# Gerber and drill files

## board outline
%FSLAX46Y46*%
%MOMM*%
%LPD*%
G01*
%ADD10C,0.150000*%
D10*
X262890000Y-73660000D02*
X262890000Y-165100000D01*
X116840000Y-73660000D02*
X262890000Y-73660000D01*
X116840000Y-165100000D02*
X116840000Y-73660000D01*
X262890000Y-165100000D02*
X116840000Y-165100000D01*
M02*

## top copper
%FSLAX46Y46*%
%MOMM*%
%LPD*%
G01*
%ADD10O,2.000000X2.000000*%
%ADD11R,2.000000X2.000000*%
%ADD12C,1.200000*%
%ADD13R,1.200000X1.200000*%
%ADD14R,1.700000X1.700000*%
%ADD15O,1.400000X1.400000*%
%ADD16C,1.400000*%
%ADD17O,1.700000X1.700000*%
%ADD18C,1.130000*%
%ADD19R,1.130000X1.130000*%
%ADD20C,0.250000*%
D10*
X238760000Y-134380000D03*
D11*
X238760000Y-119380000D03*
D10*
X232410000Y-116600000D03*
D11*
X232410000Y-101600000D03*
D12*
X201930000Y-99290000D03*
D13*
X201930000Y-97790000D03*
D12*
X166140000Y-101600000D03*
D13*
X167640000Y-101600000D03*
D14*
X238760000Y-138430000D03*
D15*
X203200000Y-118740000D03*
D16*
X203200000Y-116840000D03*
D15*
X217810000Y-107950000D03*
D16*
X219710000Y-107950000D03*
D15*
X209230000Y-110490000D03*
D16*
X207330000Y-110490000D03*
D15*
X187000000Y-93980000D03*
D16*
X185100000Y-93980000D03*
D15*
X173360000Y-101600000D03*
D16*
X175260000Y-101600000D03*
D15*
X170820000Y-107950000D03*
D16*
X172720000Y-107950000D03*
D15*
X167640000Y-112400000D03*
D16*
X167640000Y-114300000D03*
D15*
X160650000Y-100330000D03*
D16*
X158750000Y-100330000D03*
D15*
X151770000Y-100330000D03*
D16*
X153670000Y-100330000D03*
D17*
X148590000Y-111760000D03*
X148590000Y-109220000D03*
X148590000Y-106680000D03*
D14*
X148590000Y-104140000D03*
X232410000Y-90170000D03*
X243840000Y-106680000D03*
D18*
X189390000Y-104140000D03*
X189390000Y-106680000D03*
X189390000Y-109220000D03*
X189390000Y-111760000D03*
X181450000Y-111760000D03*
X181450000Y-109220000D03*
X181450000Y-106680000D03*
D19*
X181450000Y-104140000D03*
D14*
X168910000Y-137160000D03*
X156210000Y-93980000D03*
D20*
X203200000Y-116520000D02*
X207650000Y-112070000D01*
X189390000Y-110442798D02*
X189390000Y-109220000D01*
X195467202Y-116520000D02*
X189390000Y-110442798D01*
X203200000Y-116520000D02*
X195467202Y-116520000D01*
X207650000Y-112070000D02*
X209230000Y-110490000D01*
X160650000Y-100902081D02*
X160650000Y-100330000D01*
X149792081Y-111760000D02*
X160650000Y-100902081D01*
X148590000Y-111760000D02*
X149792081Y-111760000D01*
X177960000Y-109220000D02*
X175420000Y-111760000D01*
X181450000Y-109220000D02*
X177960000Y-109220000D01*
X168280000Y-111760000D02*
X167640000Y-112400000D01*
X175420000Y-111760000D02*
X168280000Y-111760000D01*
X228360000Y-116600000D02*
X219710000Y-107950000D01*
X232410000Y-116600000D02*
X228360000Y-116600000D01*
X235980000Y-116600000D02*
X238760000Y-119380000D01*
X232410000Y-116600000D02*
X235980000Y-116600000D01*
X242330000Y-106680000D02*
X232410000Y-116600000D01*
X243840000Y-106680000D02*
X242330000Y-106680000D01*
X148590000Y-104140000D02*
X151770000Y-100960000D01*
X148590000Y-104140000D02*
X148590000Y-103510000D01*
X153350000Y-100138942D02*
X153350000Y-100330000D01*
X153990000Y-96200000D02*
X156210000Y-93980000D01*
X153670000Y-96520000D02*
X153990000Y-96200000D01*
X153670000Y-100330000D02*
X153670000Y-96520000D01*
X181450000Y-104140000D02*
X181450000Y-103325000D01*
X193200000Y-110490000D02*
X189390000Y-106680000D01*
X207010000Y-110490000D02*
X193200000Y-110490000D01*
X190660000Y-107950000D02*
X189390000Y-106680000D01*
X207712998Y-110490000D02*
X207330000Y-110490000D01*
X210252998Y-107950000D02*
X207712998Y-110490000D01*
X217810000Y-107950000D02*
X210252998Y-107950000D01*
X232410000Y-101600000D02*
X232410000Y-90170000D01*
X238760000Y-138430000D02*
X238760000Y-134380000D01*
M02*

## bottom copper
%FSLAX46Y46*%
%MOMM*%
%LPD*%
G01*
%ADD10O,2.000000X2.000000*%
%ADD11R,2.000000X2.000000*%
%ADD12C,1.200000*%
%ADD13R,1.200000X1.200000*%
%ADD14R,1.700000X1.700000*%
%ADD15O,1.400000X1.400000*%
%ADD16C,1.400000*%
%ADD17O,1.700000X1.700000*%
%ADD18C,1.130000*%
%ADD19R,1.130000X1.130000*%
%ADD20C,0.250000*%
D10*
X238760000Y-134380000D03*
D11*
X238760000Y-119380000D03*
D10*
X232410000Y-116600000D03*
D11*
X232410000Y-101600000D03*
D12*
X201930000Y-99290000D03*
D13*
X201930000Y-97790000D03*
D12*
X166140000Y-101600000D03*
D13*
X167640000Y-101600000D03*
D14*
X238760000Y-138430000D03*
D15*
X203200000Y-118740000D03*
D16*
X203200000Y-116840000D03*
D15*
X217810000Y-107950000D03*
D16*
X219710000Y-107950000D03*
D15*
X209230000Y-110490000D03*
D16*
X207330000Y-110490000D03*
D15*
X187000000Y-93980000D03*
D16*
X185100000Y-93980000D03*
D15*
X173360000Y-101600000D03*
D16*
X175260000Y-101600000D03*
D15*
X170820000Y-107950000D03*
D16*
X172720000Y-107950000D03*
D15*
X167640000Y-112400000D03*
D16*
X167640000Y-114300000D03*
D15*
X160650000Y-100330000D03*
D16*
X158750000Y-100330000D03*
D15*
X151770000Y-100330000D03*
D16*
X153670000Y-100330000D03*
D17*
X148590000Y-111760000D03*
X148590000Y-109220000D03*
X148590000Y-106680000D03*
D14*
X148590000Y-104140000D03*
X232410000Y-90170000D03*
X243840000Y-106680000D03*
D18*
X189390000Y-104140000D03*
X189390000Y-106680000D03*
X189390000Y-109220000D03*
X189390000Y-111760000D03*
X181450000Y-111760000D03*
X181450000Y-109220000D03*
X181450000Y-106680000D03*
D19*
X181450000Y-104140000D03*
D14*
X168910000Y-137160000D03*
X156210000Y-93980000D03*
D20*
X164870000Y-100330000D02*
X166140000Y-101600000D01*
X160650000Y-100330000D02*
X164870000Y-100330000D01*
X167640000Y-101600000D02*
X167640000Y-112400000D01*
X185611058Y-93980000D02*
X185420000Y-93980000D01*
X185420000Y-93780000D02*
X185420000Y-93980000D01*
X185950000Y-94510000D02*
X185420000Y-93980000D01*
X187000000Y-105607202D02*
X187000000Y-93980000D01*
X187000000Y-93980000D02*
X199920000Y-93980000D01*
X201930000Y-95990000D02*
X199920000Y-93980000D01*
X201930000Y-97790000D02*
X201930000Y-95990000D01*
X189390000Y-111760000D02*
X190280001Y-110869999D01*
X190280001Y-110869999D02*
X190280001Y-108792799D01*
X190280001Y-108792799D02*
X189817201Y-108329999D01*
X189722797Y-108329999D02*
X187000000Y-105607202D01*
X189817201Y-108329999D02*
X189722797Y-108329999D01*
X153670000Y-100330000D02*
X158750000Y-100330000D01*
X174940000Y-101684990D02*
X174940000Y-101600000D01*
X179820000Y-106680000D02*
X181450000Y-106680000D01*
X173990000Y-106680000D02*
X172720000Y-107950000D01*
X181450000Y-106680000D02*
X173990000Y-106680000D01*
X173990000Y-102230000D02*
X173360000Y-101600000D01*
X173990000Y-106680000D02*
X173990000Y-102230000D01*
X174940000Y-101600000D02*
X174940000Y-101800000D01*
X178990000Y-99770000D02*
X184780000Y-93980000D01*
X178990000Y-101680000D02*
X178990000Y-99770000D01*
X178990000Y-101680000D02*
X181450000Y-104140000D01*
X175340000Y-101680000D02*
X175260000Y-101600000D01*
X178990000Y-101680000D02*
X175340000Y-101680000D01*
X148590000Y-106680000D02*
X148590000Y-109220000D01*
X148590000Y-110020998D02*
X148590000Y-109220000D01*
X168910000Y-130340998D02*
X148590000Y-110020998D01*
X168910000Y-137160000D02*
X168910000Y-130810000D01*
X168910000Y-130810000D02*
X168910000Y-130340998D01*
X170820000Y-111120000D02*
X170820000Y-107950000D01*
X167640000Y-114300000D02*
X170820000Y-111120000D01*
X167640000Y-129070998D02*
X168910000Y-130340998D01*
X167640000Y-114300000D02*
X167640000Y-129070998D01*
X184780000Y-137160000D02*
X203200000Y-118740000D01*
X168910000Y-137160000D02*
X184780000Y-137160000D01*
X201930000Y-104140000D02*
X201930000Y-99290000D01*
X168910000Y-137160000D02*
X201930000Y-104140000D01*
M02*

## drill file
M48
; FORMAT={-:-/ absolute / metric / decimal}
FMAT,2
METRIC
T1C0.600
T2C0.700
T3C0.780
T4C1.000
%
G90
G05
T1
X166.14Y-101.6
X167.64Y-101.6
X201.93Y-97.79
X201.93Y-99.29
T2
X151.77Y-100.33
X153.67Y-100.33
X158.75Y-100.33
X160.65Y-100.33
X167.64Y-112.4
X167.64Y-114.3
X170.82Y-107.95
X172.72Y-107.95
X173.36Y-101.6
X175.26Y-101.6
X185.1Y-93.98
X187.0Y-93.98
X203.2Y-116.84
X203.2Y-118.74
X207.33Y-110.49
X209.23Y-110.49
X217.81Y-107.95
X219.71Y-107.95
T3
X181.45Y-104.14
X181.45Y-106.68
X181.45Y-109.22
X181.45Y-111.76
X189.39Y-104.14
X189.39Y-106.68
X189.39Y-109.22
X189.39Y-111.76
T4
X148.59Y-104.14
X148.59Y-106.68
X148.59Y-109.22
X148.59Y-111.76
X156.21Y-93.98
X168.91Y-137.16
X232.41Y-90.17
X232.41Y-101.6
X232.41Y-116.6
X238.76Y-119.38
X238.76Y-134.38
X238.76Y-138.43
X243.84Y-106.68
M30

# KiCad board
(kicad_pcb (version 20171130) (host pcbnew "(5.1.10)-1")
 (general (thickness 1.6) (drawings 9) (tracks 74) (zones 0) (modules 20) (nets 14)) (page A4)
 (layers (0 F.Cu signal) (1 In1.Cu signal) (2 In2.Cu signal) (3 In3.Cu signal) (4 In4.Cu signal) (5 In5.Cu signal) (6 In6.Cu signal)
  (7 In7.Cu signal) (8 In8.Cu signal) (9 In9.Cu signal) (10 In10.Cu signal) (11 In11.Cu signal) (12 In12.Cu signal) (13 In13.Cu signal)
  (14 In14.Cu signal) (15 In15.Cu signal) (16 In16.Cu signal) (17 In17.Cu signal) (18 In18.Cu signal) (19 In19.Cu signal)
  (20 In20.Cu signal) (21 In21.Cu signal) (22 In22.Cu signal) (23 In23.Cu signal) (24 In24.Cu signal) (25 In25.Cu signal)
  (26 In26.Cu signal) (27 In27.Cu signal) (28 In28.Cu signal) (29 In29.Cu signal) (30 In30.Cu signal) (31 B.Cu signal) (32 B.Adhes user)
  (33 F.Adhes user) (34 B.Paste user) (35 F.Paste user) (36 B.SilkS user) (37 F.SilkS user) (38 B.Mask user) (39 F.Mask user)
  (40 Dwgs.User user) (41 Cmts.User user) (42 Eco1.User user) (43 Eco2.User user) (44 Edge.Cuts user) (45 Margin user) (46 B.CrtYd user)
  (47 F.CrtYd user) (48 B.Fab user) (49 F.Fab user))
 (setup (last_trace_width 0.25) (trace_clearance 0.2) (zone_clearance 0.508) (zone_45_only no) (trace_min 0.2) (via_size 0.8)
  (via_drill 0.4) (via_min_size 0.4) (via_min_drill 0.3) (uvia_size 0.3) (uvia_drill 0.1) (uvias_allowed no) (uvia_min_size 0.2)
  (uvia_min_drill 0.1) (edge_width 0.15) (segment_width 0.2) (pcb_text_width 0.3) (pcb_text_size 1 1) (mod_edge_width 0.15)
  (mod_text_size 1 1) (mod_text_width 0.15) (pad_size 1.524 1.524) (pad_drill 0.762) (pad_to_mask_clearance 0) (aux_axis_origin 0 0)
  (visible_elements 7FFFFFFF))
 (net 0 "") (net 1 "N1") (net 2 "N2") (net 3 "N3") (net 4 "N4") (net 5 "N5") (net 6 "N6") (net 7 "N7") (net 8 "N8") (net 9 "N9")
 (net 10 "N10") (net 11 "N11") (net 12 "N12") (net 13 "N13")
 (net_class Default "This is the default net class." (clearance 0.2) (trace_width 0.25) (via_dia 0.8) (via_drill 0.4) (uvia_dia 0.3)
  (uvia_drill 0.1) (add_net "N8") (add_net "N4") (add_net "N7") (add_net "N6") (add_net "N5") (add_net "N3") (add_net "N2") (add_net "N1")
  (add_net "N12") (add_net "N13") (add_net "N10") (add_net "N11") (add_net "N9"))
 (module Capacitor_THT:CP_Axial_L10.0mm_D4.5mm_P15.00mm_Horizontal (layer F.Cu) (at 238.76 119.38 270)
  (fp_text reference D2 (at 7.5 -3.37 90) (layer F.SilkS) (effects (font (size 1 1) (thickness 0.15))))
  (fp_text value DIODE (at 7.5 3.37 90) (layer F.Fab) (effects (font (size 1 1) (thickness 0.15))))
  (pad 2 thru_hole oval (at 15 0 270) (size 2 2) (drill 1) (layers *.Cu *.Mask) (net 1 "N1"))
  (pad 1 thru_hole rect (at 0 0 270) (size 2 2) (drill 1) (layers *.Cu *.Mask) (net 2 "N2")))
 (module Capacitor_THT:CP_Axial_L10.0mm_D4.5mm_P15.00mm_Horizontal (layer F.Cu) (at 232.41 101.6 270)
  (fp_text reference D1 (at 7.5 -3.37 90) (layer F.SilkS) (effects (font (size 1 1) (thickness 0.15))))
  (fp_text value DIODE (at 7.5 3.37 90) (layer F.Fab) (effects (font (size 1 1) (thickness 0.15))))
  (pad 2 thru_hole oval (at 15 0 270) (size 2 2) (drill 1) (layers *.Cu *.Mask) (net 2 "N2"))
  (pad 1 thru_hole rect (at 0 0 270) (size 2 2) (drill 1) (layers *.Cu *.Mask) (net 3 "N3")))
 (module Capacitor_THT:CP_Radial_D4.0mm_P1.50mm (layer B.Cu) (at 201.93 97.79 270)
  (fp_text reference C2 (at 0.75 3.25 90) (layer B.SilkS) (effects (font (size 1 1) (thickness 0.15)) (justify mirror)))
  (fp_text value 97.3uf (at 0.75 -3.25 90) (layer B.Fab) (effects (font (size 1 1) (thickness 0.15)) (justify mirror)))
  (pad 2 thru_hole circle (at 1.5 0 270) (size 1.2 1.2) (drill 0.6) (layers *.Cu *.Mask) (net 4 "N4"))
  (pad 1 thru_hole rect (at 0 0 270) (size 1.2 1.2) (drill 0.6) (layers *.Cu *.Mask) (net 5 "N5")))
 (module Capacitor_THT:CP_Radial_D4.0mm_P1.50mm (layer F.Cu) (at 167.64 101.6 180)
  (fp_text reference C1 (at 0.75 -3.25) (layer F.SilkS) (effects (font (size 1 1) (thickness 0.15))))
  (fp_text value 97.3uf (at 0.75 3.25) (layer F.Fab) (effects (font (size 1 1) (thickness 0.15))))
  (pad 2 thru_hole circle (at 1.5 0 180) (size 1.2 1.2) (drill 0.6) (layers *.Cu *.Mask) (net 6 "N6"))
  (pad 1 thru_hole rect (at 0 0 180) (size 1.2 1.2) (drill 0.6) (layers *.Cu *.Mask) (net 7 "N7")))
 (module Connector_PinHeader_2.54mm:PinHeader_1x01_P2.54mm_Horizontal (layer F.Cu) (at 238.76 138.43 270)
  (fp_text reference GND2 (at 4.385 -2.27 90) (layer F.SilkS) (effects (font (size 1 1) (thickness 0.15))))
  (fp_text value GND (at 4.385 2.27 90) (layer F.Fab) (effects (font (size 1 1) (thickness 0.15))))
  (pad 1 thru_hole rect (at 0 0 270) (size 1.7 1.7) (drill 1) (layers *.Cu *.Mask) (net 1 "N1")))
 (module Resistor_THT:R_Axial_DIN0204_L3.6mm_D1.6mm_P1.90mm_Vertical (layer F.Cu) (at 203.2 116.84 270)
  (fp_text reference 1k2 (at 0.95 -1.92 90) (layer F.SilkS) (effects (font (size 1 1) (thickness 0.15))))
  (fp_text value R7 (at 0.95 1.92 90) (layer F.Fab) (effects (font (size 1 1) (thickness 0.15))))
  (pad 2 thru_hole oval (at 1.9 0 270) (size 1.4 1.4) (drill 0.7) (layers *.Cu *.Mask) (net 4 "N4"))
  (pad 1 thru_hole circle (at 0 0 270) (size 1.4 1.4) (drill 0.7) (layers *.Cu *.Mask) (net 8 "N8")))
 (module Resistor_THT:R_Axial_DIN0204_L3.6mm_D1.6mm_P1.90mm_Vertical (layer F.Cu) (at 219.71 107.95 180)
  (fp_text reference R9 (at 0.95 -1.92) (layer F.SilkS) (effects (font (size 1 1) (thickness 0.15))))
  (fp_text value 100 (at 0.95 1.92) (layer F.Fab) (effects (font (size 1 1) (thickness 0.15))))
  (pad 2 thru_hole oval (at 1.9 0 180) (size 1.4 1.4) (drill 0.7) (layers *.Cu *.Mask) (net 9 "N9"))
  (pad 1 thru_hole circle (at 0 0 180) (size 1.4 1.4) (drill 0.7) (layers *.Cu *.Mask) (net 2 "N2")))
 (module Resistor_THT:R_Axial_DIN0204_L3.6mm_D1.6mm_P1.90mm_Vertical (layer F.Cu) (at 207.33 110.49)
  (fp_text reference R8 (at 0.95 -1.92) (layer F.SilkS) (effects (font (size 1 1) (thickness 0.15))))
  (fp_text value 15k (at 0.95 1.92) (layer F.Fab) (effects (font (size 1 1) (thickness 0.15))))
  (pad 2 thru_hole oval (at 1.9 0) (size 1.4 1.4) (drill 0.7) (layers *.Cu *.Mask) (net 8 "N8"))
  (pad 1 thru_hole circle (at 0 0) (size 1.4 1.4) (drill 0.7) (layers *.Cu *.Mask) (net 9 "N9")))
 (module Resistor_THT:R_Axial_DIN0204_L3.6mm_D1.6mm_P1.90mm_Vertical (layer B.Cu) (at 185.1 93.98)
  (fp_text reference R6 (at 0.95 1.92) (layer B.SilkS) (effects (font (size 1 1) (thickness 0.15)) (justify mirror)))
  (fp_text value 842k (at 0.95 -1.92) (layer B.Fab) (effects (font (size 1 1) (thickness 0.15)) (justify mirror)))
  (pad 2 thru_hole oval (at 1.9 0) (size 1.4 1.4) (drill 0.7) (layers *.Cu *.Mask) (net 5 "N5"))
  (pad 1 thru_hole circle (at 0 0) (size 1.4 1.4) (drill 0.7) (layers *.Cu *.Mask) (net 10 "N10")))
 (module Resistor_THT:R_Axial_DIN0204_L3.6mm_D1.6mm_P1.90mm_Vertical (layer B.Cu) (at 175.26 101.6 180)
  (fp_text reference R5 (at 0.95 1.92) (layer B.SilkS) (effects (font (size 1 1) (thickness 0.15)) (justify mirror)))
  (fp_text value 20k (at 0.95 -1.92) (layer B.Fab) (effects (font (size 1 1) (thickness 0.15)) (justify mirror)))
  (pad 2 thru_hole oval (at 1.9 0 180) (size 1.4 1.4) (drill 0.7) (layers *.Cu *.Mask) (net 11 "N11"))
  (pad 1 thru_hole circle (at 0 0 180) (size 1.4 1.4) (drill 0.7) (layers *.Cu *.Mask) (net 10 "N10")))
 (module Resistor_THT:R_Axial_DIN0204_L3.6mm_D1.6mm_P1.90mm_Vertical (layer B.Cu) (at 172.72 107.95 180)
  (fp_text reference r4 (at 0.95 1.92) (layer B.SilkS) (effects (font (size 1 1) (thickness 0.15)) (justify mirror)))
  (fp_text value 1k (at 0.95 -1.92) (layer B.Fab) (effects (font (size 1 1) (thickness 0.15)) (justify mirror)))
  (pad 2 thru_hole oval (at 1.9 0 180) (size 1.4 1.4) (drill 0.7) (layers *.Cu *.Mask) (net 4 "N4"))
  (pad 1 thru_hole circle (at 0 0 180) (size 1.4 1.4) (drill 0.7) (layers *.Cu *.Mask) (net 11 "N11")))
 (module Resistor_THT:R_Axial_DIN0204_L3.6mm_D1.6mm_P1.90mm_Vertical (layer F.Cu) (at 167.64 114.3 90)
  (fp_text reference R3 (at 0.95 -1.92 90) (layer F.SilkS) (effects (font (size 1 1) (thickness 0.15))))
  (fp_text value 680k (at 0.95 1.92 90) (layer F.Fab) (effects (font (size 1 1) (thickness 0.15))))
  (pad 2 thru_hole oval (at 1.9 0 90) (size 1.4 1.4) (drill 0.7) (layers *.Cu *.Mask) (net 7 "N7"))
  (pad 1 thru_hole circle (at 0 0 90) (size 1.4 1.4) (drill 0.7) (layers *.Cu *.Mask) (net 4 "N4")))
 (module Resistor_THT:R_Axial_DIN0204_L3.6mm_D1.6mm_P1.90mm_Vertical (layer F.Cu) (at 158.75 100.33)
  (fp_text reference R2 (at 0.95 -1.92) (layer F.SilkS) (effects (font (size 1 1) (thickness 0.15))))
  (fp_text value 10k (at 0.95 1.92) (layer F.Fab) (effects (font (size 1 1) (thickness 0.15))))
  (pad 2 thru_hole oval (at 1.9 0) (size 1.4 1.4) (drill 0.7) (layers *.Cu *.Mask) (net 6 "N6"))
  (pad 1 thru_hole circle (at 0 0) (size 1.4 1.4) (drill 0.7) (layers *.Cu *.Mask) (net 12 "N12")))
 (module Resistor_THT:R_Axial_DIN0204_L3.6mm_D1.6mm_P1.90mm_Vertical (layer F.Cu) (at 153.67 100.33 180)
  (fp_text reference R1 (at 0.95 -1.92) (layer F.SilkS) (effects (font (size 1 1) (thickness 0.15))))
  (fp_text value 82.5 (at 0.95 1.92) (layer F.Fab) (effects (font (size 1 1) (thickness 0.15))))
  (pad 2 thru_hole oval (at 1.9 0 180) (size 1.4 1.4) (drill 0.7) (layers *.Cu *.Mask) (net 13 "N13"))
  (pad 1 thru_hole circle (at 0 0 180) (size 1.4 1.4) (drill 0.7) (layers *.Cu *.Mask) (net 12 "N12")))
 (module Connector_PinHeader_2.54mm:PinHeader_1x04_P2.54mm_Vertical (layer F.Cu) (at 148.59 104.14)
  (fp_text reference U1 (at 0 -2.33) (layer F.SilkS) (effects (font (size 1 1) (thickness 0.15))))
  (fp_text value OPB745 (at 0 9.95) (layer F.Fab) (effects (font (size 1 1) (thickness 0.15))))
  (pad 4 thru_hole oval (at 0 7.62) (size 1.7 1.7) (drill 1) (layers *.Cu *.Mask) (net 6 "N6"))
  (pad 3 thru_hole oval (at 0 5.08) (size 1.7 1.7) (drill 1) (layers *.Cu *.Mask) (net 4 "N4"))
  (pad 2 thru_hole oval (at 0 2.54) (size 1.7 1.7) (drill 1) (layers *.Cu *.Mask) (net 4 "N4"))
  (pad 1 thru_hole rect (at 0 0) (size 1.7 1.7) (drill 1) (layers *.Cu *.Mask) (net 13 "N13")))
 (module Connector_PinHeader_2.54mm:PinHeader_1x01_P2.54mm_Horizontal (layer F.Cu) (at 232.41 90.17 90)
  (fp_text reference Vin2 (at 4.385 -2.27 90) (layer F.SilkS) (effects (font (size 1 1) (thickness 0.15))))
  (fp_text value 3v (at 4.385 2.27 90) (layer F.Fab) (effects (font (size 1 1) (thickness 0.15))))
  (pad 1 thru_hole rect (at 0 0 90) (size 1.7 1.7) (drill 1) (layers *.Cu *.Mask) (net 3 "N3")))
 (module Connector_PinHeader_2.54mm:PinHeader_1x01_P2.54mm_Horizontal (layer F.Cu) (at 243.84 106.68)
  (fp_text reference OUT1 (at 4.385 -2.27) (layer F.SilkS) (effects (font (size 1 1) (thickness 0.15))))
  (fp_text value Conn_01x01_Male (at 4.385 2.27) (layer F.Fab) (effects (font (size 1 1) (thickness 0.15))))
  (pad 1 thru_hole rect (at 0 0) (size 1.7 1.7) (drill 1) (layers *.Cu *.Mask) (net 2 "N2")))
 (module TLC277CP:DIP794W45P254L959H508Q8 (layer F.Cu) (at 185.42 107.95)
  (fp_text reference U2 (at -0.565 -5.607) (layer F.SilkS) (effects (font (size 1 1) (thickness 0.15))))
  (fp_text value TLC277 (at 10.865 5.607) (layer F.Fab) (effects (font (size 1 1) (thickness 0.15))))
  (pad 8 thru_hole circle (at 3.97 -3.81) (size 1.13 1.13) (drill 0.78) (layers *.Cu *.Mask))
  (pad 7 thru_hole circle (at 3.97 -1.27) (size 1.13 1.13) (drill 0.78) (layers *.Cu *.Mask) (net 9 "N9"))
  (pad 6 thru_hole circle (at 3.97 1.27) (size 1.13 1.13) (drill 0.78) (layers *.Cu *.Mask) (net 8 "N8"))
  (pad 5 thru_hole circle (at 3.97 3.81) (size 1.13 1.13) (drill 0.78) (layers *.Cu *.Mask) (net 5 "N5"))
  (pad 4 thru_hole circle (at -3.97 3.81) (size 1.13 1.13) (drill 0.78) (layers *.Cu *.Mask))
  (pad 3 thru_hole circle (at -3.97 1.27) (size 1.13 1.13) (drill 0.78) (layers *.Cu *.Mask) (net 7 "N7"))
  (pad 2 thru_hole circle (at -3.97 -1.27) (size 1.13 1.13) (drill 0.78) (layers *.Cu *.Mask) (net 11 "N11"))
  (pad 1 thru_hole rect (at -3.97 -3.81) (size 1.13 1.13) (drill 0.78) (layers *.Cu *.Mask) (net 10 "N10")))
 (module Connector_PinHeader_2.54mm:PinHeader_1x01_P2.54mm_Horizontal (layer F.Cu) (at 168.91 137.16 270)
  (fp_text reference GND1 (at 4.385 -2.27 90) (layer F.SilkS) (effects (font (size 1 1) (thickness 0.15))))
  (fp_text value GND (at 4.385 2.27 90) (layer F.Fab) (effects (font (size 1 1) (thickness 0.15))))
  (pad 1 thru_hole rect (at 0 0 270) (size 1.7 1.7) (drill 1) (layers *.Cu *.Mask) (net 4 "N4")))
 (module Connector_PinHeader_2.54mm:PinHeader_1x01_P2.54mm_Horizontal (layer F.Cu) (at 156.21 93.98 90)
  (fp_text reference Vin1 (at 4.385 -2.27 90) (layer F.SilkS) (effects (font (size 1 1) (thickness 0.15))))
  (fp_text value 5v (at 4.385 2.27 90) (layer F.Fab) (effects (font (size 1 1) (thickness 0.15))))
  (pad 1 thru_hole rect (at 0 0 90) (size 1.7 1.7) (drill 1) (layers *.Cu *.Mask) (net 12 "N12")))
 (gr_line (start 262.89 73.66) (end 262.89 165.1) (layer Edge.Cuts) (width 0.15))
 (gr_line (start 116.84 73.66) (end 262.89 73.66) (layer Edge.Cuts) (width 0.15))
 (gr_line (start 116.84 165.1) (end 116.84 73.66) (layer Edge.Cuts) (width 0.15))
 (gr_line (start 262.89 165.1) (end 116.84 165.1) (layer Edge.Cuts) (width 0.15))
 (segment (start 203.2 116.52) (end 207.65 112.07) (width 0.25) (layer F.Cu) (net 8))
 (segment (start 189.39 110.442798) (end 189.39 109.22) (width 0.25) (layer F.Cu) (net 8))
 (segment (start 195.467202 116.52) (end 189.39 110.442798) (width 0.25) (layer F.Cu) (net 8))
 (segment (start 203.2 116.52) (end 195.467202 116.52) (width 0.25) (layer F.Cu) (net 8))
 (segment (start 207.65 112.07) (end 209.23 110.49) (width 0.25) (layer F.Cu) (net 8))
 (segment (start 164.87 100.33) (end 166.14 101.6) (width 0.25) (layer B.Cu) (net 6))
 (segment (start 160.65 100.33) (end 164.87 100.33) (width 0.25) (layer B.Cu) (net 6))
 (segment (start 160.65 100.902081) (end 160.65 100.33) (width 0.25) (layer F.Cu) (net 6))
 (segment (start 149.792081 111.76) (end 160.65 100.902081) (width 0.25) (layer F.Cu) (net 6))
 (segment (start 148.59 111.76) (end 149.792081 111.76) (width 0.25) (layer F.Cu) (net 6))
 (segment (start 177.96 109.22) (end 175.42 111.76) (width 0.25) (layer F.Cu) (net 7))
 (segment (start 181.45 109.22) (end 177.96 109.22) (width 0.25) (layer F.Cu) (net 7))
 (segment (start 168.28 111.76) (end 167.64 112.4) (width 0.25) (layer F.Cu) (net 7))
 (segment (start 175.42 111.76) (end 168.28 111.76) (width 0.25) (layer F.Cu) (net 7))
 (segment (start 167.64 101.6) (end 167.64 112.4) (width 0.25) (layer B.Cu) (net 7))
 (segment (start 185.611058 93.98) (end 185.42 93.98) (width 0.25) (layer B.Cu) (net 10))
 (segment (start 185.42 93.78) (end 185.42 93.98) (width 0.25) (layer B.Cu) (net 10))
 (segment (start 185.95 94.51) (end 185.42 93.98) (width 0.25) (layer B.Cu) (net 10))
 (segment (start 187 105.607202) (end 187 93.98) (width 0.25) (layer B.Cu) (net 5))
 (segment (start 187 93.98) (end 199.92 93.98) (width 0.25) (layer B.Cu) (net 5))
 (segment (start 201.93 95.99) (end 199.92 93.98) (width 0.25) (layer B.Cu) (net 5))
 (segment (start 201.93 97.79) (end 201.93 95.99) (width 0.25) (layer B.Cu) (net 5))
 (segment (start 189.39 111.76) (end 190.280001 110.869999) (width 0.25) (layer B.Cu) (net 5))
 (segment (start 190.280001 110.869999) (end 190.280001 108.792799) (width 0.25) (layer B.Cu) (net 5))
 (segment (start 190.280001 108.792799) (end 189.817201 108.329999) (width 0.25) (layer B.Cu) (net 5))
 (segment (start 189.722797 108.329999) (end 187 105.607202) (width 0.25) (layer B.Cu) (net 5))
 (segment (start 189.817201 108.329999) (end 189.722797 108.329999) (width 0.25) (layer B.Cu) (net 5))
 (segment (start 228.36 116.6) (end 219.71 107.95) (width 0.25) (layer F.Cu) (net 2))
 (segment (start 232.41 116.6) (end 228.36 116.6) (width 0.25) (layer F.Cu) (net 2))
 (segment (start 235.98 116.6) (end 238.76 119.38) (width 0.25) (layer F.Cu) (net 2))
 (segment (start 232.41 116.6) (end 235.98 116.6) (width 0.25) (layer F.Cu) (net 2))
 (segment (start 242.33 106.68) (end 232.41 116.6) (width 0.25) (layer F.Cu) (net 2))
 (segment (start 243.84 106.68) (end 242.33 106.68) (width 0.25) (layer F.Cu) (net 2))
 (segment (start 148.59 104.14) (end 151.77 100.96) (width 0.25) (layer F.Cu) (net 13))
 (segment (start 148.59 104.14) (end 148.59 103.51) (width 0.25) (layer F.Cu) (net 13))
 (segment (start 153.35 100.138942) (end 153.35 100.33) (width 0.25) (layer F.Cu) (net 12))
 (segment (start 153.99 96.2) (end 156.21 93.98) (width 0.25) (layer F.Cu) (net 12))
 (segment (start 153.67 96.52) (end 153.99 96.2) (width 0.25) (layer F.Cu) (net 12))
 (segment (start 153.67 100.33) (end 153.67 96.52) (width 0.25) (layer F.Cu) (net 12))
 (segment (start 153.67 100.33) (end 158.75 100.33) (width 0.25) (layer B.Cu) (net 12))
 (segment (start 174.94 101.68499) (end 174.94 101.6) (width 0.25) (layer B.Cu) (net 10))
 (segment (start 179.82 106.68) (end 181.45 106.68) (width 0.25) (layer B.Cu) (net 11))
 (segment (start 173.99 106.68) (end 172.72 107.95) (width 0.25) (layer B.Cu) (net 11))
 (segment (start 181.45 106.68) (end 173.99 106.68) (width 0.25) (layer B.Cu) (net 11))
 (segment (start 173.99 102.23) (end 173.36 101.6) (width 0.25) (layer B.Cu) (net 11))
 (segment (start 173.99 106.68) (end 173.99 102.23) (width 0.25) (layer B.Cu) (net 11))
 (segment (start 174.94 101.6) (end 174.94 101.8) (width 0.25) (layer B.Cu) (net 10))
 (segment (start 181.45 104.14) (end 181.45 103.325) (width 0.25) (layer F.Cu) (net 10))
 (segment (start 178.99 99.77) (end 184.78 93.98) (width 0.25) (layer B.Cu) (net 10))
 (segment (start 178.99 101.68) (end 178.99 99.77) (width 0.25) (layer B.Cu) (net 10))
 (segment (start 178.99 101.68) (end 181.45 104.14) (width 0.25) (layer B.Cu) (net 10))
 (segment (start 175.34 101.68) (end 175.26 101.6) (width 0.25) (layer B.Cu) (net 10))
 (segment (start 178.99 101.68) (end 175.34 101.68) (width 0.25) (layer B.Cu) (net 10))
 (segment (start 193.2 110.49) (end 189.39 106.68) (width 0.25) (layer F.Cu) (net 9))
 (segment (start 207.01 110.49) (end 193.2 110.49) (width 0.25) (layer F.Cu) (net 9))
 (segment (start 190.66 107.95) (end 189.39 106.68) (width 0.25) (layer F.Cu) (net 9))
 (segment (start 207.712998 110.49) (end 207.33 110.49) (width 0.25) (layer F.Cu) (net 9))
 (segment (start 210.252998 107.95) (end 207.712998 110.49) (width 0.25) (layer F.Cu) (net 9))
 (segment (start 217.81 107.95) (end 210.252998 107.95) (width 0.25) (layer F.Cu) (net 9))
 (segment (start 148.59 106.68) (end 148.59 109.22) (width 0.25) (layer B.Cu) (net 4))
 (segment (start 148.59 110.020998) (end 148.59 109.22) (width 0.25) (layer B.Cu) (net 4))
 (segment (start 168.91 130.340998) (end 148.59 110.020998) (width 0.25) (layer B.Cu) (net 4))
 (segment (start 168.91 137.16) (end 168.91 130.81) (width 0.25) (layer B.Cu) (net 4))
 (segment (start 168.91 130.81) (end 168.91 130.340998) (width 0.25) (layer B.Cu) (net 4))
 (segment (start 170.82 111.12) (end 170.82 107.95) (width 0.25) (layer B.Cu) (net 4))
 (segment (start 167.64 114.3) (end 170.82 111.12) (width 0.25) (layer B.Cu) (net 4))
 (segment (start 167.64 129.070998) (end 168.91 130.340998) (width 0.25) (layer B.Cu) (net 4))
 (segment (start 167.64 114.3) (end 167.64 129.070998) (width 0.25) (layer B.Cu) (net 4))
 (segment (start 184.78 137.16) (end 203.2 118.74) (width 0.25) (layer B.Cu) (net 4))
 (segment (start 168.91 137.16) (end 184.78 137.16) (width 0.25) (layer B.Cu) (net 4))
 (segment (start 201.93 104.14) (end 201.93 99.29) (width 0.25) (layer B.Cu) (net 4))
 (segment (start 168.91 137.16) (end 201.93 104.14) (width 0.25) (layer B.Cu) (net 4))
 (segment (start 232.41 101.6) (end 232.41 90.17) (width 0.25) (layer F.Cu) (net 3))
 (segment (start 238.76 138.43) (end 238.76 134.38) (width 0.25) (layer F.Cu) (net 1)))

